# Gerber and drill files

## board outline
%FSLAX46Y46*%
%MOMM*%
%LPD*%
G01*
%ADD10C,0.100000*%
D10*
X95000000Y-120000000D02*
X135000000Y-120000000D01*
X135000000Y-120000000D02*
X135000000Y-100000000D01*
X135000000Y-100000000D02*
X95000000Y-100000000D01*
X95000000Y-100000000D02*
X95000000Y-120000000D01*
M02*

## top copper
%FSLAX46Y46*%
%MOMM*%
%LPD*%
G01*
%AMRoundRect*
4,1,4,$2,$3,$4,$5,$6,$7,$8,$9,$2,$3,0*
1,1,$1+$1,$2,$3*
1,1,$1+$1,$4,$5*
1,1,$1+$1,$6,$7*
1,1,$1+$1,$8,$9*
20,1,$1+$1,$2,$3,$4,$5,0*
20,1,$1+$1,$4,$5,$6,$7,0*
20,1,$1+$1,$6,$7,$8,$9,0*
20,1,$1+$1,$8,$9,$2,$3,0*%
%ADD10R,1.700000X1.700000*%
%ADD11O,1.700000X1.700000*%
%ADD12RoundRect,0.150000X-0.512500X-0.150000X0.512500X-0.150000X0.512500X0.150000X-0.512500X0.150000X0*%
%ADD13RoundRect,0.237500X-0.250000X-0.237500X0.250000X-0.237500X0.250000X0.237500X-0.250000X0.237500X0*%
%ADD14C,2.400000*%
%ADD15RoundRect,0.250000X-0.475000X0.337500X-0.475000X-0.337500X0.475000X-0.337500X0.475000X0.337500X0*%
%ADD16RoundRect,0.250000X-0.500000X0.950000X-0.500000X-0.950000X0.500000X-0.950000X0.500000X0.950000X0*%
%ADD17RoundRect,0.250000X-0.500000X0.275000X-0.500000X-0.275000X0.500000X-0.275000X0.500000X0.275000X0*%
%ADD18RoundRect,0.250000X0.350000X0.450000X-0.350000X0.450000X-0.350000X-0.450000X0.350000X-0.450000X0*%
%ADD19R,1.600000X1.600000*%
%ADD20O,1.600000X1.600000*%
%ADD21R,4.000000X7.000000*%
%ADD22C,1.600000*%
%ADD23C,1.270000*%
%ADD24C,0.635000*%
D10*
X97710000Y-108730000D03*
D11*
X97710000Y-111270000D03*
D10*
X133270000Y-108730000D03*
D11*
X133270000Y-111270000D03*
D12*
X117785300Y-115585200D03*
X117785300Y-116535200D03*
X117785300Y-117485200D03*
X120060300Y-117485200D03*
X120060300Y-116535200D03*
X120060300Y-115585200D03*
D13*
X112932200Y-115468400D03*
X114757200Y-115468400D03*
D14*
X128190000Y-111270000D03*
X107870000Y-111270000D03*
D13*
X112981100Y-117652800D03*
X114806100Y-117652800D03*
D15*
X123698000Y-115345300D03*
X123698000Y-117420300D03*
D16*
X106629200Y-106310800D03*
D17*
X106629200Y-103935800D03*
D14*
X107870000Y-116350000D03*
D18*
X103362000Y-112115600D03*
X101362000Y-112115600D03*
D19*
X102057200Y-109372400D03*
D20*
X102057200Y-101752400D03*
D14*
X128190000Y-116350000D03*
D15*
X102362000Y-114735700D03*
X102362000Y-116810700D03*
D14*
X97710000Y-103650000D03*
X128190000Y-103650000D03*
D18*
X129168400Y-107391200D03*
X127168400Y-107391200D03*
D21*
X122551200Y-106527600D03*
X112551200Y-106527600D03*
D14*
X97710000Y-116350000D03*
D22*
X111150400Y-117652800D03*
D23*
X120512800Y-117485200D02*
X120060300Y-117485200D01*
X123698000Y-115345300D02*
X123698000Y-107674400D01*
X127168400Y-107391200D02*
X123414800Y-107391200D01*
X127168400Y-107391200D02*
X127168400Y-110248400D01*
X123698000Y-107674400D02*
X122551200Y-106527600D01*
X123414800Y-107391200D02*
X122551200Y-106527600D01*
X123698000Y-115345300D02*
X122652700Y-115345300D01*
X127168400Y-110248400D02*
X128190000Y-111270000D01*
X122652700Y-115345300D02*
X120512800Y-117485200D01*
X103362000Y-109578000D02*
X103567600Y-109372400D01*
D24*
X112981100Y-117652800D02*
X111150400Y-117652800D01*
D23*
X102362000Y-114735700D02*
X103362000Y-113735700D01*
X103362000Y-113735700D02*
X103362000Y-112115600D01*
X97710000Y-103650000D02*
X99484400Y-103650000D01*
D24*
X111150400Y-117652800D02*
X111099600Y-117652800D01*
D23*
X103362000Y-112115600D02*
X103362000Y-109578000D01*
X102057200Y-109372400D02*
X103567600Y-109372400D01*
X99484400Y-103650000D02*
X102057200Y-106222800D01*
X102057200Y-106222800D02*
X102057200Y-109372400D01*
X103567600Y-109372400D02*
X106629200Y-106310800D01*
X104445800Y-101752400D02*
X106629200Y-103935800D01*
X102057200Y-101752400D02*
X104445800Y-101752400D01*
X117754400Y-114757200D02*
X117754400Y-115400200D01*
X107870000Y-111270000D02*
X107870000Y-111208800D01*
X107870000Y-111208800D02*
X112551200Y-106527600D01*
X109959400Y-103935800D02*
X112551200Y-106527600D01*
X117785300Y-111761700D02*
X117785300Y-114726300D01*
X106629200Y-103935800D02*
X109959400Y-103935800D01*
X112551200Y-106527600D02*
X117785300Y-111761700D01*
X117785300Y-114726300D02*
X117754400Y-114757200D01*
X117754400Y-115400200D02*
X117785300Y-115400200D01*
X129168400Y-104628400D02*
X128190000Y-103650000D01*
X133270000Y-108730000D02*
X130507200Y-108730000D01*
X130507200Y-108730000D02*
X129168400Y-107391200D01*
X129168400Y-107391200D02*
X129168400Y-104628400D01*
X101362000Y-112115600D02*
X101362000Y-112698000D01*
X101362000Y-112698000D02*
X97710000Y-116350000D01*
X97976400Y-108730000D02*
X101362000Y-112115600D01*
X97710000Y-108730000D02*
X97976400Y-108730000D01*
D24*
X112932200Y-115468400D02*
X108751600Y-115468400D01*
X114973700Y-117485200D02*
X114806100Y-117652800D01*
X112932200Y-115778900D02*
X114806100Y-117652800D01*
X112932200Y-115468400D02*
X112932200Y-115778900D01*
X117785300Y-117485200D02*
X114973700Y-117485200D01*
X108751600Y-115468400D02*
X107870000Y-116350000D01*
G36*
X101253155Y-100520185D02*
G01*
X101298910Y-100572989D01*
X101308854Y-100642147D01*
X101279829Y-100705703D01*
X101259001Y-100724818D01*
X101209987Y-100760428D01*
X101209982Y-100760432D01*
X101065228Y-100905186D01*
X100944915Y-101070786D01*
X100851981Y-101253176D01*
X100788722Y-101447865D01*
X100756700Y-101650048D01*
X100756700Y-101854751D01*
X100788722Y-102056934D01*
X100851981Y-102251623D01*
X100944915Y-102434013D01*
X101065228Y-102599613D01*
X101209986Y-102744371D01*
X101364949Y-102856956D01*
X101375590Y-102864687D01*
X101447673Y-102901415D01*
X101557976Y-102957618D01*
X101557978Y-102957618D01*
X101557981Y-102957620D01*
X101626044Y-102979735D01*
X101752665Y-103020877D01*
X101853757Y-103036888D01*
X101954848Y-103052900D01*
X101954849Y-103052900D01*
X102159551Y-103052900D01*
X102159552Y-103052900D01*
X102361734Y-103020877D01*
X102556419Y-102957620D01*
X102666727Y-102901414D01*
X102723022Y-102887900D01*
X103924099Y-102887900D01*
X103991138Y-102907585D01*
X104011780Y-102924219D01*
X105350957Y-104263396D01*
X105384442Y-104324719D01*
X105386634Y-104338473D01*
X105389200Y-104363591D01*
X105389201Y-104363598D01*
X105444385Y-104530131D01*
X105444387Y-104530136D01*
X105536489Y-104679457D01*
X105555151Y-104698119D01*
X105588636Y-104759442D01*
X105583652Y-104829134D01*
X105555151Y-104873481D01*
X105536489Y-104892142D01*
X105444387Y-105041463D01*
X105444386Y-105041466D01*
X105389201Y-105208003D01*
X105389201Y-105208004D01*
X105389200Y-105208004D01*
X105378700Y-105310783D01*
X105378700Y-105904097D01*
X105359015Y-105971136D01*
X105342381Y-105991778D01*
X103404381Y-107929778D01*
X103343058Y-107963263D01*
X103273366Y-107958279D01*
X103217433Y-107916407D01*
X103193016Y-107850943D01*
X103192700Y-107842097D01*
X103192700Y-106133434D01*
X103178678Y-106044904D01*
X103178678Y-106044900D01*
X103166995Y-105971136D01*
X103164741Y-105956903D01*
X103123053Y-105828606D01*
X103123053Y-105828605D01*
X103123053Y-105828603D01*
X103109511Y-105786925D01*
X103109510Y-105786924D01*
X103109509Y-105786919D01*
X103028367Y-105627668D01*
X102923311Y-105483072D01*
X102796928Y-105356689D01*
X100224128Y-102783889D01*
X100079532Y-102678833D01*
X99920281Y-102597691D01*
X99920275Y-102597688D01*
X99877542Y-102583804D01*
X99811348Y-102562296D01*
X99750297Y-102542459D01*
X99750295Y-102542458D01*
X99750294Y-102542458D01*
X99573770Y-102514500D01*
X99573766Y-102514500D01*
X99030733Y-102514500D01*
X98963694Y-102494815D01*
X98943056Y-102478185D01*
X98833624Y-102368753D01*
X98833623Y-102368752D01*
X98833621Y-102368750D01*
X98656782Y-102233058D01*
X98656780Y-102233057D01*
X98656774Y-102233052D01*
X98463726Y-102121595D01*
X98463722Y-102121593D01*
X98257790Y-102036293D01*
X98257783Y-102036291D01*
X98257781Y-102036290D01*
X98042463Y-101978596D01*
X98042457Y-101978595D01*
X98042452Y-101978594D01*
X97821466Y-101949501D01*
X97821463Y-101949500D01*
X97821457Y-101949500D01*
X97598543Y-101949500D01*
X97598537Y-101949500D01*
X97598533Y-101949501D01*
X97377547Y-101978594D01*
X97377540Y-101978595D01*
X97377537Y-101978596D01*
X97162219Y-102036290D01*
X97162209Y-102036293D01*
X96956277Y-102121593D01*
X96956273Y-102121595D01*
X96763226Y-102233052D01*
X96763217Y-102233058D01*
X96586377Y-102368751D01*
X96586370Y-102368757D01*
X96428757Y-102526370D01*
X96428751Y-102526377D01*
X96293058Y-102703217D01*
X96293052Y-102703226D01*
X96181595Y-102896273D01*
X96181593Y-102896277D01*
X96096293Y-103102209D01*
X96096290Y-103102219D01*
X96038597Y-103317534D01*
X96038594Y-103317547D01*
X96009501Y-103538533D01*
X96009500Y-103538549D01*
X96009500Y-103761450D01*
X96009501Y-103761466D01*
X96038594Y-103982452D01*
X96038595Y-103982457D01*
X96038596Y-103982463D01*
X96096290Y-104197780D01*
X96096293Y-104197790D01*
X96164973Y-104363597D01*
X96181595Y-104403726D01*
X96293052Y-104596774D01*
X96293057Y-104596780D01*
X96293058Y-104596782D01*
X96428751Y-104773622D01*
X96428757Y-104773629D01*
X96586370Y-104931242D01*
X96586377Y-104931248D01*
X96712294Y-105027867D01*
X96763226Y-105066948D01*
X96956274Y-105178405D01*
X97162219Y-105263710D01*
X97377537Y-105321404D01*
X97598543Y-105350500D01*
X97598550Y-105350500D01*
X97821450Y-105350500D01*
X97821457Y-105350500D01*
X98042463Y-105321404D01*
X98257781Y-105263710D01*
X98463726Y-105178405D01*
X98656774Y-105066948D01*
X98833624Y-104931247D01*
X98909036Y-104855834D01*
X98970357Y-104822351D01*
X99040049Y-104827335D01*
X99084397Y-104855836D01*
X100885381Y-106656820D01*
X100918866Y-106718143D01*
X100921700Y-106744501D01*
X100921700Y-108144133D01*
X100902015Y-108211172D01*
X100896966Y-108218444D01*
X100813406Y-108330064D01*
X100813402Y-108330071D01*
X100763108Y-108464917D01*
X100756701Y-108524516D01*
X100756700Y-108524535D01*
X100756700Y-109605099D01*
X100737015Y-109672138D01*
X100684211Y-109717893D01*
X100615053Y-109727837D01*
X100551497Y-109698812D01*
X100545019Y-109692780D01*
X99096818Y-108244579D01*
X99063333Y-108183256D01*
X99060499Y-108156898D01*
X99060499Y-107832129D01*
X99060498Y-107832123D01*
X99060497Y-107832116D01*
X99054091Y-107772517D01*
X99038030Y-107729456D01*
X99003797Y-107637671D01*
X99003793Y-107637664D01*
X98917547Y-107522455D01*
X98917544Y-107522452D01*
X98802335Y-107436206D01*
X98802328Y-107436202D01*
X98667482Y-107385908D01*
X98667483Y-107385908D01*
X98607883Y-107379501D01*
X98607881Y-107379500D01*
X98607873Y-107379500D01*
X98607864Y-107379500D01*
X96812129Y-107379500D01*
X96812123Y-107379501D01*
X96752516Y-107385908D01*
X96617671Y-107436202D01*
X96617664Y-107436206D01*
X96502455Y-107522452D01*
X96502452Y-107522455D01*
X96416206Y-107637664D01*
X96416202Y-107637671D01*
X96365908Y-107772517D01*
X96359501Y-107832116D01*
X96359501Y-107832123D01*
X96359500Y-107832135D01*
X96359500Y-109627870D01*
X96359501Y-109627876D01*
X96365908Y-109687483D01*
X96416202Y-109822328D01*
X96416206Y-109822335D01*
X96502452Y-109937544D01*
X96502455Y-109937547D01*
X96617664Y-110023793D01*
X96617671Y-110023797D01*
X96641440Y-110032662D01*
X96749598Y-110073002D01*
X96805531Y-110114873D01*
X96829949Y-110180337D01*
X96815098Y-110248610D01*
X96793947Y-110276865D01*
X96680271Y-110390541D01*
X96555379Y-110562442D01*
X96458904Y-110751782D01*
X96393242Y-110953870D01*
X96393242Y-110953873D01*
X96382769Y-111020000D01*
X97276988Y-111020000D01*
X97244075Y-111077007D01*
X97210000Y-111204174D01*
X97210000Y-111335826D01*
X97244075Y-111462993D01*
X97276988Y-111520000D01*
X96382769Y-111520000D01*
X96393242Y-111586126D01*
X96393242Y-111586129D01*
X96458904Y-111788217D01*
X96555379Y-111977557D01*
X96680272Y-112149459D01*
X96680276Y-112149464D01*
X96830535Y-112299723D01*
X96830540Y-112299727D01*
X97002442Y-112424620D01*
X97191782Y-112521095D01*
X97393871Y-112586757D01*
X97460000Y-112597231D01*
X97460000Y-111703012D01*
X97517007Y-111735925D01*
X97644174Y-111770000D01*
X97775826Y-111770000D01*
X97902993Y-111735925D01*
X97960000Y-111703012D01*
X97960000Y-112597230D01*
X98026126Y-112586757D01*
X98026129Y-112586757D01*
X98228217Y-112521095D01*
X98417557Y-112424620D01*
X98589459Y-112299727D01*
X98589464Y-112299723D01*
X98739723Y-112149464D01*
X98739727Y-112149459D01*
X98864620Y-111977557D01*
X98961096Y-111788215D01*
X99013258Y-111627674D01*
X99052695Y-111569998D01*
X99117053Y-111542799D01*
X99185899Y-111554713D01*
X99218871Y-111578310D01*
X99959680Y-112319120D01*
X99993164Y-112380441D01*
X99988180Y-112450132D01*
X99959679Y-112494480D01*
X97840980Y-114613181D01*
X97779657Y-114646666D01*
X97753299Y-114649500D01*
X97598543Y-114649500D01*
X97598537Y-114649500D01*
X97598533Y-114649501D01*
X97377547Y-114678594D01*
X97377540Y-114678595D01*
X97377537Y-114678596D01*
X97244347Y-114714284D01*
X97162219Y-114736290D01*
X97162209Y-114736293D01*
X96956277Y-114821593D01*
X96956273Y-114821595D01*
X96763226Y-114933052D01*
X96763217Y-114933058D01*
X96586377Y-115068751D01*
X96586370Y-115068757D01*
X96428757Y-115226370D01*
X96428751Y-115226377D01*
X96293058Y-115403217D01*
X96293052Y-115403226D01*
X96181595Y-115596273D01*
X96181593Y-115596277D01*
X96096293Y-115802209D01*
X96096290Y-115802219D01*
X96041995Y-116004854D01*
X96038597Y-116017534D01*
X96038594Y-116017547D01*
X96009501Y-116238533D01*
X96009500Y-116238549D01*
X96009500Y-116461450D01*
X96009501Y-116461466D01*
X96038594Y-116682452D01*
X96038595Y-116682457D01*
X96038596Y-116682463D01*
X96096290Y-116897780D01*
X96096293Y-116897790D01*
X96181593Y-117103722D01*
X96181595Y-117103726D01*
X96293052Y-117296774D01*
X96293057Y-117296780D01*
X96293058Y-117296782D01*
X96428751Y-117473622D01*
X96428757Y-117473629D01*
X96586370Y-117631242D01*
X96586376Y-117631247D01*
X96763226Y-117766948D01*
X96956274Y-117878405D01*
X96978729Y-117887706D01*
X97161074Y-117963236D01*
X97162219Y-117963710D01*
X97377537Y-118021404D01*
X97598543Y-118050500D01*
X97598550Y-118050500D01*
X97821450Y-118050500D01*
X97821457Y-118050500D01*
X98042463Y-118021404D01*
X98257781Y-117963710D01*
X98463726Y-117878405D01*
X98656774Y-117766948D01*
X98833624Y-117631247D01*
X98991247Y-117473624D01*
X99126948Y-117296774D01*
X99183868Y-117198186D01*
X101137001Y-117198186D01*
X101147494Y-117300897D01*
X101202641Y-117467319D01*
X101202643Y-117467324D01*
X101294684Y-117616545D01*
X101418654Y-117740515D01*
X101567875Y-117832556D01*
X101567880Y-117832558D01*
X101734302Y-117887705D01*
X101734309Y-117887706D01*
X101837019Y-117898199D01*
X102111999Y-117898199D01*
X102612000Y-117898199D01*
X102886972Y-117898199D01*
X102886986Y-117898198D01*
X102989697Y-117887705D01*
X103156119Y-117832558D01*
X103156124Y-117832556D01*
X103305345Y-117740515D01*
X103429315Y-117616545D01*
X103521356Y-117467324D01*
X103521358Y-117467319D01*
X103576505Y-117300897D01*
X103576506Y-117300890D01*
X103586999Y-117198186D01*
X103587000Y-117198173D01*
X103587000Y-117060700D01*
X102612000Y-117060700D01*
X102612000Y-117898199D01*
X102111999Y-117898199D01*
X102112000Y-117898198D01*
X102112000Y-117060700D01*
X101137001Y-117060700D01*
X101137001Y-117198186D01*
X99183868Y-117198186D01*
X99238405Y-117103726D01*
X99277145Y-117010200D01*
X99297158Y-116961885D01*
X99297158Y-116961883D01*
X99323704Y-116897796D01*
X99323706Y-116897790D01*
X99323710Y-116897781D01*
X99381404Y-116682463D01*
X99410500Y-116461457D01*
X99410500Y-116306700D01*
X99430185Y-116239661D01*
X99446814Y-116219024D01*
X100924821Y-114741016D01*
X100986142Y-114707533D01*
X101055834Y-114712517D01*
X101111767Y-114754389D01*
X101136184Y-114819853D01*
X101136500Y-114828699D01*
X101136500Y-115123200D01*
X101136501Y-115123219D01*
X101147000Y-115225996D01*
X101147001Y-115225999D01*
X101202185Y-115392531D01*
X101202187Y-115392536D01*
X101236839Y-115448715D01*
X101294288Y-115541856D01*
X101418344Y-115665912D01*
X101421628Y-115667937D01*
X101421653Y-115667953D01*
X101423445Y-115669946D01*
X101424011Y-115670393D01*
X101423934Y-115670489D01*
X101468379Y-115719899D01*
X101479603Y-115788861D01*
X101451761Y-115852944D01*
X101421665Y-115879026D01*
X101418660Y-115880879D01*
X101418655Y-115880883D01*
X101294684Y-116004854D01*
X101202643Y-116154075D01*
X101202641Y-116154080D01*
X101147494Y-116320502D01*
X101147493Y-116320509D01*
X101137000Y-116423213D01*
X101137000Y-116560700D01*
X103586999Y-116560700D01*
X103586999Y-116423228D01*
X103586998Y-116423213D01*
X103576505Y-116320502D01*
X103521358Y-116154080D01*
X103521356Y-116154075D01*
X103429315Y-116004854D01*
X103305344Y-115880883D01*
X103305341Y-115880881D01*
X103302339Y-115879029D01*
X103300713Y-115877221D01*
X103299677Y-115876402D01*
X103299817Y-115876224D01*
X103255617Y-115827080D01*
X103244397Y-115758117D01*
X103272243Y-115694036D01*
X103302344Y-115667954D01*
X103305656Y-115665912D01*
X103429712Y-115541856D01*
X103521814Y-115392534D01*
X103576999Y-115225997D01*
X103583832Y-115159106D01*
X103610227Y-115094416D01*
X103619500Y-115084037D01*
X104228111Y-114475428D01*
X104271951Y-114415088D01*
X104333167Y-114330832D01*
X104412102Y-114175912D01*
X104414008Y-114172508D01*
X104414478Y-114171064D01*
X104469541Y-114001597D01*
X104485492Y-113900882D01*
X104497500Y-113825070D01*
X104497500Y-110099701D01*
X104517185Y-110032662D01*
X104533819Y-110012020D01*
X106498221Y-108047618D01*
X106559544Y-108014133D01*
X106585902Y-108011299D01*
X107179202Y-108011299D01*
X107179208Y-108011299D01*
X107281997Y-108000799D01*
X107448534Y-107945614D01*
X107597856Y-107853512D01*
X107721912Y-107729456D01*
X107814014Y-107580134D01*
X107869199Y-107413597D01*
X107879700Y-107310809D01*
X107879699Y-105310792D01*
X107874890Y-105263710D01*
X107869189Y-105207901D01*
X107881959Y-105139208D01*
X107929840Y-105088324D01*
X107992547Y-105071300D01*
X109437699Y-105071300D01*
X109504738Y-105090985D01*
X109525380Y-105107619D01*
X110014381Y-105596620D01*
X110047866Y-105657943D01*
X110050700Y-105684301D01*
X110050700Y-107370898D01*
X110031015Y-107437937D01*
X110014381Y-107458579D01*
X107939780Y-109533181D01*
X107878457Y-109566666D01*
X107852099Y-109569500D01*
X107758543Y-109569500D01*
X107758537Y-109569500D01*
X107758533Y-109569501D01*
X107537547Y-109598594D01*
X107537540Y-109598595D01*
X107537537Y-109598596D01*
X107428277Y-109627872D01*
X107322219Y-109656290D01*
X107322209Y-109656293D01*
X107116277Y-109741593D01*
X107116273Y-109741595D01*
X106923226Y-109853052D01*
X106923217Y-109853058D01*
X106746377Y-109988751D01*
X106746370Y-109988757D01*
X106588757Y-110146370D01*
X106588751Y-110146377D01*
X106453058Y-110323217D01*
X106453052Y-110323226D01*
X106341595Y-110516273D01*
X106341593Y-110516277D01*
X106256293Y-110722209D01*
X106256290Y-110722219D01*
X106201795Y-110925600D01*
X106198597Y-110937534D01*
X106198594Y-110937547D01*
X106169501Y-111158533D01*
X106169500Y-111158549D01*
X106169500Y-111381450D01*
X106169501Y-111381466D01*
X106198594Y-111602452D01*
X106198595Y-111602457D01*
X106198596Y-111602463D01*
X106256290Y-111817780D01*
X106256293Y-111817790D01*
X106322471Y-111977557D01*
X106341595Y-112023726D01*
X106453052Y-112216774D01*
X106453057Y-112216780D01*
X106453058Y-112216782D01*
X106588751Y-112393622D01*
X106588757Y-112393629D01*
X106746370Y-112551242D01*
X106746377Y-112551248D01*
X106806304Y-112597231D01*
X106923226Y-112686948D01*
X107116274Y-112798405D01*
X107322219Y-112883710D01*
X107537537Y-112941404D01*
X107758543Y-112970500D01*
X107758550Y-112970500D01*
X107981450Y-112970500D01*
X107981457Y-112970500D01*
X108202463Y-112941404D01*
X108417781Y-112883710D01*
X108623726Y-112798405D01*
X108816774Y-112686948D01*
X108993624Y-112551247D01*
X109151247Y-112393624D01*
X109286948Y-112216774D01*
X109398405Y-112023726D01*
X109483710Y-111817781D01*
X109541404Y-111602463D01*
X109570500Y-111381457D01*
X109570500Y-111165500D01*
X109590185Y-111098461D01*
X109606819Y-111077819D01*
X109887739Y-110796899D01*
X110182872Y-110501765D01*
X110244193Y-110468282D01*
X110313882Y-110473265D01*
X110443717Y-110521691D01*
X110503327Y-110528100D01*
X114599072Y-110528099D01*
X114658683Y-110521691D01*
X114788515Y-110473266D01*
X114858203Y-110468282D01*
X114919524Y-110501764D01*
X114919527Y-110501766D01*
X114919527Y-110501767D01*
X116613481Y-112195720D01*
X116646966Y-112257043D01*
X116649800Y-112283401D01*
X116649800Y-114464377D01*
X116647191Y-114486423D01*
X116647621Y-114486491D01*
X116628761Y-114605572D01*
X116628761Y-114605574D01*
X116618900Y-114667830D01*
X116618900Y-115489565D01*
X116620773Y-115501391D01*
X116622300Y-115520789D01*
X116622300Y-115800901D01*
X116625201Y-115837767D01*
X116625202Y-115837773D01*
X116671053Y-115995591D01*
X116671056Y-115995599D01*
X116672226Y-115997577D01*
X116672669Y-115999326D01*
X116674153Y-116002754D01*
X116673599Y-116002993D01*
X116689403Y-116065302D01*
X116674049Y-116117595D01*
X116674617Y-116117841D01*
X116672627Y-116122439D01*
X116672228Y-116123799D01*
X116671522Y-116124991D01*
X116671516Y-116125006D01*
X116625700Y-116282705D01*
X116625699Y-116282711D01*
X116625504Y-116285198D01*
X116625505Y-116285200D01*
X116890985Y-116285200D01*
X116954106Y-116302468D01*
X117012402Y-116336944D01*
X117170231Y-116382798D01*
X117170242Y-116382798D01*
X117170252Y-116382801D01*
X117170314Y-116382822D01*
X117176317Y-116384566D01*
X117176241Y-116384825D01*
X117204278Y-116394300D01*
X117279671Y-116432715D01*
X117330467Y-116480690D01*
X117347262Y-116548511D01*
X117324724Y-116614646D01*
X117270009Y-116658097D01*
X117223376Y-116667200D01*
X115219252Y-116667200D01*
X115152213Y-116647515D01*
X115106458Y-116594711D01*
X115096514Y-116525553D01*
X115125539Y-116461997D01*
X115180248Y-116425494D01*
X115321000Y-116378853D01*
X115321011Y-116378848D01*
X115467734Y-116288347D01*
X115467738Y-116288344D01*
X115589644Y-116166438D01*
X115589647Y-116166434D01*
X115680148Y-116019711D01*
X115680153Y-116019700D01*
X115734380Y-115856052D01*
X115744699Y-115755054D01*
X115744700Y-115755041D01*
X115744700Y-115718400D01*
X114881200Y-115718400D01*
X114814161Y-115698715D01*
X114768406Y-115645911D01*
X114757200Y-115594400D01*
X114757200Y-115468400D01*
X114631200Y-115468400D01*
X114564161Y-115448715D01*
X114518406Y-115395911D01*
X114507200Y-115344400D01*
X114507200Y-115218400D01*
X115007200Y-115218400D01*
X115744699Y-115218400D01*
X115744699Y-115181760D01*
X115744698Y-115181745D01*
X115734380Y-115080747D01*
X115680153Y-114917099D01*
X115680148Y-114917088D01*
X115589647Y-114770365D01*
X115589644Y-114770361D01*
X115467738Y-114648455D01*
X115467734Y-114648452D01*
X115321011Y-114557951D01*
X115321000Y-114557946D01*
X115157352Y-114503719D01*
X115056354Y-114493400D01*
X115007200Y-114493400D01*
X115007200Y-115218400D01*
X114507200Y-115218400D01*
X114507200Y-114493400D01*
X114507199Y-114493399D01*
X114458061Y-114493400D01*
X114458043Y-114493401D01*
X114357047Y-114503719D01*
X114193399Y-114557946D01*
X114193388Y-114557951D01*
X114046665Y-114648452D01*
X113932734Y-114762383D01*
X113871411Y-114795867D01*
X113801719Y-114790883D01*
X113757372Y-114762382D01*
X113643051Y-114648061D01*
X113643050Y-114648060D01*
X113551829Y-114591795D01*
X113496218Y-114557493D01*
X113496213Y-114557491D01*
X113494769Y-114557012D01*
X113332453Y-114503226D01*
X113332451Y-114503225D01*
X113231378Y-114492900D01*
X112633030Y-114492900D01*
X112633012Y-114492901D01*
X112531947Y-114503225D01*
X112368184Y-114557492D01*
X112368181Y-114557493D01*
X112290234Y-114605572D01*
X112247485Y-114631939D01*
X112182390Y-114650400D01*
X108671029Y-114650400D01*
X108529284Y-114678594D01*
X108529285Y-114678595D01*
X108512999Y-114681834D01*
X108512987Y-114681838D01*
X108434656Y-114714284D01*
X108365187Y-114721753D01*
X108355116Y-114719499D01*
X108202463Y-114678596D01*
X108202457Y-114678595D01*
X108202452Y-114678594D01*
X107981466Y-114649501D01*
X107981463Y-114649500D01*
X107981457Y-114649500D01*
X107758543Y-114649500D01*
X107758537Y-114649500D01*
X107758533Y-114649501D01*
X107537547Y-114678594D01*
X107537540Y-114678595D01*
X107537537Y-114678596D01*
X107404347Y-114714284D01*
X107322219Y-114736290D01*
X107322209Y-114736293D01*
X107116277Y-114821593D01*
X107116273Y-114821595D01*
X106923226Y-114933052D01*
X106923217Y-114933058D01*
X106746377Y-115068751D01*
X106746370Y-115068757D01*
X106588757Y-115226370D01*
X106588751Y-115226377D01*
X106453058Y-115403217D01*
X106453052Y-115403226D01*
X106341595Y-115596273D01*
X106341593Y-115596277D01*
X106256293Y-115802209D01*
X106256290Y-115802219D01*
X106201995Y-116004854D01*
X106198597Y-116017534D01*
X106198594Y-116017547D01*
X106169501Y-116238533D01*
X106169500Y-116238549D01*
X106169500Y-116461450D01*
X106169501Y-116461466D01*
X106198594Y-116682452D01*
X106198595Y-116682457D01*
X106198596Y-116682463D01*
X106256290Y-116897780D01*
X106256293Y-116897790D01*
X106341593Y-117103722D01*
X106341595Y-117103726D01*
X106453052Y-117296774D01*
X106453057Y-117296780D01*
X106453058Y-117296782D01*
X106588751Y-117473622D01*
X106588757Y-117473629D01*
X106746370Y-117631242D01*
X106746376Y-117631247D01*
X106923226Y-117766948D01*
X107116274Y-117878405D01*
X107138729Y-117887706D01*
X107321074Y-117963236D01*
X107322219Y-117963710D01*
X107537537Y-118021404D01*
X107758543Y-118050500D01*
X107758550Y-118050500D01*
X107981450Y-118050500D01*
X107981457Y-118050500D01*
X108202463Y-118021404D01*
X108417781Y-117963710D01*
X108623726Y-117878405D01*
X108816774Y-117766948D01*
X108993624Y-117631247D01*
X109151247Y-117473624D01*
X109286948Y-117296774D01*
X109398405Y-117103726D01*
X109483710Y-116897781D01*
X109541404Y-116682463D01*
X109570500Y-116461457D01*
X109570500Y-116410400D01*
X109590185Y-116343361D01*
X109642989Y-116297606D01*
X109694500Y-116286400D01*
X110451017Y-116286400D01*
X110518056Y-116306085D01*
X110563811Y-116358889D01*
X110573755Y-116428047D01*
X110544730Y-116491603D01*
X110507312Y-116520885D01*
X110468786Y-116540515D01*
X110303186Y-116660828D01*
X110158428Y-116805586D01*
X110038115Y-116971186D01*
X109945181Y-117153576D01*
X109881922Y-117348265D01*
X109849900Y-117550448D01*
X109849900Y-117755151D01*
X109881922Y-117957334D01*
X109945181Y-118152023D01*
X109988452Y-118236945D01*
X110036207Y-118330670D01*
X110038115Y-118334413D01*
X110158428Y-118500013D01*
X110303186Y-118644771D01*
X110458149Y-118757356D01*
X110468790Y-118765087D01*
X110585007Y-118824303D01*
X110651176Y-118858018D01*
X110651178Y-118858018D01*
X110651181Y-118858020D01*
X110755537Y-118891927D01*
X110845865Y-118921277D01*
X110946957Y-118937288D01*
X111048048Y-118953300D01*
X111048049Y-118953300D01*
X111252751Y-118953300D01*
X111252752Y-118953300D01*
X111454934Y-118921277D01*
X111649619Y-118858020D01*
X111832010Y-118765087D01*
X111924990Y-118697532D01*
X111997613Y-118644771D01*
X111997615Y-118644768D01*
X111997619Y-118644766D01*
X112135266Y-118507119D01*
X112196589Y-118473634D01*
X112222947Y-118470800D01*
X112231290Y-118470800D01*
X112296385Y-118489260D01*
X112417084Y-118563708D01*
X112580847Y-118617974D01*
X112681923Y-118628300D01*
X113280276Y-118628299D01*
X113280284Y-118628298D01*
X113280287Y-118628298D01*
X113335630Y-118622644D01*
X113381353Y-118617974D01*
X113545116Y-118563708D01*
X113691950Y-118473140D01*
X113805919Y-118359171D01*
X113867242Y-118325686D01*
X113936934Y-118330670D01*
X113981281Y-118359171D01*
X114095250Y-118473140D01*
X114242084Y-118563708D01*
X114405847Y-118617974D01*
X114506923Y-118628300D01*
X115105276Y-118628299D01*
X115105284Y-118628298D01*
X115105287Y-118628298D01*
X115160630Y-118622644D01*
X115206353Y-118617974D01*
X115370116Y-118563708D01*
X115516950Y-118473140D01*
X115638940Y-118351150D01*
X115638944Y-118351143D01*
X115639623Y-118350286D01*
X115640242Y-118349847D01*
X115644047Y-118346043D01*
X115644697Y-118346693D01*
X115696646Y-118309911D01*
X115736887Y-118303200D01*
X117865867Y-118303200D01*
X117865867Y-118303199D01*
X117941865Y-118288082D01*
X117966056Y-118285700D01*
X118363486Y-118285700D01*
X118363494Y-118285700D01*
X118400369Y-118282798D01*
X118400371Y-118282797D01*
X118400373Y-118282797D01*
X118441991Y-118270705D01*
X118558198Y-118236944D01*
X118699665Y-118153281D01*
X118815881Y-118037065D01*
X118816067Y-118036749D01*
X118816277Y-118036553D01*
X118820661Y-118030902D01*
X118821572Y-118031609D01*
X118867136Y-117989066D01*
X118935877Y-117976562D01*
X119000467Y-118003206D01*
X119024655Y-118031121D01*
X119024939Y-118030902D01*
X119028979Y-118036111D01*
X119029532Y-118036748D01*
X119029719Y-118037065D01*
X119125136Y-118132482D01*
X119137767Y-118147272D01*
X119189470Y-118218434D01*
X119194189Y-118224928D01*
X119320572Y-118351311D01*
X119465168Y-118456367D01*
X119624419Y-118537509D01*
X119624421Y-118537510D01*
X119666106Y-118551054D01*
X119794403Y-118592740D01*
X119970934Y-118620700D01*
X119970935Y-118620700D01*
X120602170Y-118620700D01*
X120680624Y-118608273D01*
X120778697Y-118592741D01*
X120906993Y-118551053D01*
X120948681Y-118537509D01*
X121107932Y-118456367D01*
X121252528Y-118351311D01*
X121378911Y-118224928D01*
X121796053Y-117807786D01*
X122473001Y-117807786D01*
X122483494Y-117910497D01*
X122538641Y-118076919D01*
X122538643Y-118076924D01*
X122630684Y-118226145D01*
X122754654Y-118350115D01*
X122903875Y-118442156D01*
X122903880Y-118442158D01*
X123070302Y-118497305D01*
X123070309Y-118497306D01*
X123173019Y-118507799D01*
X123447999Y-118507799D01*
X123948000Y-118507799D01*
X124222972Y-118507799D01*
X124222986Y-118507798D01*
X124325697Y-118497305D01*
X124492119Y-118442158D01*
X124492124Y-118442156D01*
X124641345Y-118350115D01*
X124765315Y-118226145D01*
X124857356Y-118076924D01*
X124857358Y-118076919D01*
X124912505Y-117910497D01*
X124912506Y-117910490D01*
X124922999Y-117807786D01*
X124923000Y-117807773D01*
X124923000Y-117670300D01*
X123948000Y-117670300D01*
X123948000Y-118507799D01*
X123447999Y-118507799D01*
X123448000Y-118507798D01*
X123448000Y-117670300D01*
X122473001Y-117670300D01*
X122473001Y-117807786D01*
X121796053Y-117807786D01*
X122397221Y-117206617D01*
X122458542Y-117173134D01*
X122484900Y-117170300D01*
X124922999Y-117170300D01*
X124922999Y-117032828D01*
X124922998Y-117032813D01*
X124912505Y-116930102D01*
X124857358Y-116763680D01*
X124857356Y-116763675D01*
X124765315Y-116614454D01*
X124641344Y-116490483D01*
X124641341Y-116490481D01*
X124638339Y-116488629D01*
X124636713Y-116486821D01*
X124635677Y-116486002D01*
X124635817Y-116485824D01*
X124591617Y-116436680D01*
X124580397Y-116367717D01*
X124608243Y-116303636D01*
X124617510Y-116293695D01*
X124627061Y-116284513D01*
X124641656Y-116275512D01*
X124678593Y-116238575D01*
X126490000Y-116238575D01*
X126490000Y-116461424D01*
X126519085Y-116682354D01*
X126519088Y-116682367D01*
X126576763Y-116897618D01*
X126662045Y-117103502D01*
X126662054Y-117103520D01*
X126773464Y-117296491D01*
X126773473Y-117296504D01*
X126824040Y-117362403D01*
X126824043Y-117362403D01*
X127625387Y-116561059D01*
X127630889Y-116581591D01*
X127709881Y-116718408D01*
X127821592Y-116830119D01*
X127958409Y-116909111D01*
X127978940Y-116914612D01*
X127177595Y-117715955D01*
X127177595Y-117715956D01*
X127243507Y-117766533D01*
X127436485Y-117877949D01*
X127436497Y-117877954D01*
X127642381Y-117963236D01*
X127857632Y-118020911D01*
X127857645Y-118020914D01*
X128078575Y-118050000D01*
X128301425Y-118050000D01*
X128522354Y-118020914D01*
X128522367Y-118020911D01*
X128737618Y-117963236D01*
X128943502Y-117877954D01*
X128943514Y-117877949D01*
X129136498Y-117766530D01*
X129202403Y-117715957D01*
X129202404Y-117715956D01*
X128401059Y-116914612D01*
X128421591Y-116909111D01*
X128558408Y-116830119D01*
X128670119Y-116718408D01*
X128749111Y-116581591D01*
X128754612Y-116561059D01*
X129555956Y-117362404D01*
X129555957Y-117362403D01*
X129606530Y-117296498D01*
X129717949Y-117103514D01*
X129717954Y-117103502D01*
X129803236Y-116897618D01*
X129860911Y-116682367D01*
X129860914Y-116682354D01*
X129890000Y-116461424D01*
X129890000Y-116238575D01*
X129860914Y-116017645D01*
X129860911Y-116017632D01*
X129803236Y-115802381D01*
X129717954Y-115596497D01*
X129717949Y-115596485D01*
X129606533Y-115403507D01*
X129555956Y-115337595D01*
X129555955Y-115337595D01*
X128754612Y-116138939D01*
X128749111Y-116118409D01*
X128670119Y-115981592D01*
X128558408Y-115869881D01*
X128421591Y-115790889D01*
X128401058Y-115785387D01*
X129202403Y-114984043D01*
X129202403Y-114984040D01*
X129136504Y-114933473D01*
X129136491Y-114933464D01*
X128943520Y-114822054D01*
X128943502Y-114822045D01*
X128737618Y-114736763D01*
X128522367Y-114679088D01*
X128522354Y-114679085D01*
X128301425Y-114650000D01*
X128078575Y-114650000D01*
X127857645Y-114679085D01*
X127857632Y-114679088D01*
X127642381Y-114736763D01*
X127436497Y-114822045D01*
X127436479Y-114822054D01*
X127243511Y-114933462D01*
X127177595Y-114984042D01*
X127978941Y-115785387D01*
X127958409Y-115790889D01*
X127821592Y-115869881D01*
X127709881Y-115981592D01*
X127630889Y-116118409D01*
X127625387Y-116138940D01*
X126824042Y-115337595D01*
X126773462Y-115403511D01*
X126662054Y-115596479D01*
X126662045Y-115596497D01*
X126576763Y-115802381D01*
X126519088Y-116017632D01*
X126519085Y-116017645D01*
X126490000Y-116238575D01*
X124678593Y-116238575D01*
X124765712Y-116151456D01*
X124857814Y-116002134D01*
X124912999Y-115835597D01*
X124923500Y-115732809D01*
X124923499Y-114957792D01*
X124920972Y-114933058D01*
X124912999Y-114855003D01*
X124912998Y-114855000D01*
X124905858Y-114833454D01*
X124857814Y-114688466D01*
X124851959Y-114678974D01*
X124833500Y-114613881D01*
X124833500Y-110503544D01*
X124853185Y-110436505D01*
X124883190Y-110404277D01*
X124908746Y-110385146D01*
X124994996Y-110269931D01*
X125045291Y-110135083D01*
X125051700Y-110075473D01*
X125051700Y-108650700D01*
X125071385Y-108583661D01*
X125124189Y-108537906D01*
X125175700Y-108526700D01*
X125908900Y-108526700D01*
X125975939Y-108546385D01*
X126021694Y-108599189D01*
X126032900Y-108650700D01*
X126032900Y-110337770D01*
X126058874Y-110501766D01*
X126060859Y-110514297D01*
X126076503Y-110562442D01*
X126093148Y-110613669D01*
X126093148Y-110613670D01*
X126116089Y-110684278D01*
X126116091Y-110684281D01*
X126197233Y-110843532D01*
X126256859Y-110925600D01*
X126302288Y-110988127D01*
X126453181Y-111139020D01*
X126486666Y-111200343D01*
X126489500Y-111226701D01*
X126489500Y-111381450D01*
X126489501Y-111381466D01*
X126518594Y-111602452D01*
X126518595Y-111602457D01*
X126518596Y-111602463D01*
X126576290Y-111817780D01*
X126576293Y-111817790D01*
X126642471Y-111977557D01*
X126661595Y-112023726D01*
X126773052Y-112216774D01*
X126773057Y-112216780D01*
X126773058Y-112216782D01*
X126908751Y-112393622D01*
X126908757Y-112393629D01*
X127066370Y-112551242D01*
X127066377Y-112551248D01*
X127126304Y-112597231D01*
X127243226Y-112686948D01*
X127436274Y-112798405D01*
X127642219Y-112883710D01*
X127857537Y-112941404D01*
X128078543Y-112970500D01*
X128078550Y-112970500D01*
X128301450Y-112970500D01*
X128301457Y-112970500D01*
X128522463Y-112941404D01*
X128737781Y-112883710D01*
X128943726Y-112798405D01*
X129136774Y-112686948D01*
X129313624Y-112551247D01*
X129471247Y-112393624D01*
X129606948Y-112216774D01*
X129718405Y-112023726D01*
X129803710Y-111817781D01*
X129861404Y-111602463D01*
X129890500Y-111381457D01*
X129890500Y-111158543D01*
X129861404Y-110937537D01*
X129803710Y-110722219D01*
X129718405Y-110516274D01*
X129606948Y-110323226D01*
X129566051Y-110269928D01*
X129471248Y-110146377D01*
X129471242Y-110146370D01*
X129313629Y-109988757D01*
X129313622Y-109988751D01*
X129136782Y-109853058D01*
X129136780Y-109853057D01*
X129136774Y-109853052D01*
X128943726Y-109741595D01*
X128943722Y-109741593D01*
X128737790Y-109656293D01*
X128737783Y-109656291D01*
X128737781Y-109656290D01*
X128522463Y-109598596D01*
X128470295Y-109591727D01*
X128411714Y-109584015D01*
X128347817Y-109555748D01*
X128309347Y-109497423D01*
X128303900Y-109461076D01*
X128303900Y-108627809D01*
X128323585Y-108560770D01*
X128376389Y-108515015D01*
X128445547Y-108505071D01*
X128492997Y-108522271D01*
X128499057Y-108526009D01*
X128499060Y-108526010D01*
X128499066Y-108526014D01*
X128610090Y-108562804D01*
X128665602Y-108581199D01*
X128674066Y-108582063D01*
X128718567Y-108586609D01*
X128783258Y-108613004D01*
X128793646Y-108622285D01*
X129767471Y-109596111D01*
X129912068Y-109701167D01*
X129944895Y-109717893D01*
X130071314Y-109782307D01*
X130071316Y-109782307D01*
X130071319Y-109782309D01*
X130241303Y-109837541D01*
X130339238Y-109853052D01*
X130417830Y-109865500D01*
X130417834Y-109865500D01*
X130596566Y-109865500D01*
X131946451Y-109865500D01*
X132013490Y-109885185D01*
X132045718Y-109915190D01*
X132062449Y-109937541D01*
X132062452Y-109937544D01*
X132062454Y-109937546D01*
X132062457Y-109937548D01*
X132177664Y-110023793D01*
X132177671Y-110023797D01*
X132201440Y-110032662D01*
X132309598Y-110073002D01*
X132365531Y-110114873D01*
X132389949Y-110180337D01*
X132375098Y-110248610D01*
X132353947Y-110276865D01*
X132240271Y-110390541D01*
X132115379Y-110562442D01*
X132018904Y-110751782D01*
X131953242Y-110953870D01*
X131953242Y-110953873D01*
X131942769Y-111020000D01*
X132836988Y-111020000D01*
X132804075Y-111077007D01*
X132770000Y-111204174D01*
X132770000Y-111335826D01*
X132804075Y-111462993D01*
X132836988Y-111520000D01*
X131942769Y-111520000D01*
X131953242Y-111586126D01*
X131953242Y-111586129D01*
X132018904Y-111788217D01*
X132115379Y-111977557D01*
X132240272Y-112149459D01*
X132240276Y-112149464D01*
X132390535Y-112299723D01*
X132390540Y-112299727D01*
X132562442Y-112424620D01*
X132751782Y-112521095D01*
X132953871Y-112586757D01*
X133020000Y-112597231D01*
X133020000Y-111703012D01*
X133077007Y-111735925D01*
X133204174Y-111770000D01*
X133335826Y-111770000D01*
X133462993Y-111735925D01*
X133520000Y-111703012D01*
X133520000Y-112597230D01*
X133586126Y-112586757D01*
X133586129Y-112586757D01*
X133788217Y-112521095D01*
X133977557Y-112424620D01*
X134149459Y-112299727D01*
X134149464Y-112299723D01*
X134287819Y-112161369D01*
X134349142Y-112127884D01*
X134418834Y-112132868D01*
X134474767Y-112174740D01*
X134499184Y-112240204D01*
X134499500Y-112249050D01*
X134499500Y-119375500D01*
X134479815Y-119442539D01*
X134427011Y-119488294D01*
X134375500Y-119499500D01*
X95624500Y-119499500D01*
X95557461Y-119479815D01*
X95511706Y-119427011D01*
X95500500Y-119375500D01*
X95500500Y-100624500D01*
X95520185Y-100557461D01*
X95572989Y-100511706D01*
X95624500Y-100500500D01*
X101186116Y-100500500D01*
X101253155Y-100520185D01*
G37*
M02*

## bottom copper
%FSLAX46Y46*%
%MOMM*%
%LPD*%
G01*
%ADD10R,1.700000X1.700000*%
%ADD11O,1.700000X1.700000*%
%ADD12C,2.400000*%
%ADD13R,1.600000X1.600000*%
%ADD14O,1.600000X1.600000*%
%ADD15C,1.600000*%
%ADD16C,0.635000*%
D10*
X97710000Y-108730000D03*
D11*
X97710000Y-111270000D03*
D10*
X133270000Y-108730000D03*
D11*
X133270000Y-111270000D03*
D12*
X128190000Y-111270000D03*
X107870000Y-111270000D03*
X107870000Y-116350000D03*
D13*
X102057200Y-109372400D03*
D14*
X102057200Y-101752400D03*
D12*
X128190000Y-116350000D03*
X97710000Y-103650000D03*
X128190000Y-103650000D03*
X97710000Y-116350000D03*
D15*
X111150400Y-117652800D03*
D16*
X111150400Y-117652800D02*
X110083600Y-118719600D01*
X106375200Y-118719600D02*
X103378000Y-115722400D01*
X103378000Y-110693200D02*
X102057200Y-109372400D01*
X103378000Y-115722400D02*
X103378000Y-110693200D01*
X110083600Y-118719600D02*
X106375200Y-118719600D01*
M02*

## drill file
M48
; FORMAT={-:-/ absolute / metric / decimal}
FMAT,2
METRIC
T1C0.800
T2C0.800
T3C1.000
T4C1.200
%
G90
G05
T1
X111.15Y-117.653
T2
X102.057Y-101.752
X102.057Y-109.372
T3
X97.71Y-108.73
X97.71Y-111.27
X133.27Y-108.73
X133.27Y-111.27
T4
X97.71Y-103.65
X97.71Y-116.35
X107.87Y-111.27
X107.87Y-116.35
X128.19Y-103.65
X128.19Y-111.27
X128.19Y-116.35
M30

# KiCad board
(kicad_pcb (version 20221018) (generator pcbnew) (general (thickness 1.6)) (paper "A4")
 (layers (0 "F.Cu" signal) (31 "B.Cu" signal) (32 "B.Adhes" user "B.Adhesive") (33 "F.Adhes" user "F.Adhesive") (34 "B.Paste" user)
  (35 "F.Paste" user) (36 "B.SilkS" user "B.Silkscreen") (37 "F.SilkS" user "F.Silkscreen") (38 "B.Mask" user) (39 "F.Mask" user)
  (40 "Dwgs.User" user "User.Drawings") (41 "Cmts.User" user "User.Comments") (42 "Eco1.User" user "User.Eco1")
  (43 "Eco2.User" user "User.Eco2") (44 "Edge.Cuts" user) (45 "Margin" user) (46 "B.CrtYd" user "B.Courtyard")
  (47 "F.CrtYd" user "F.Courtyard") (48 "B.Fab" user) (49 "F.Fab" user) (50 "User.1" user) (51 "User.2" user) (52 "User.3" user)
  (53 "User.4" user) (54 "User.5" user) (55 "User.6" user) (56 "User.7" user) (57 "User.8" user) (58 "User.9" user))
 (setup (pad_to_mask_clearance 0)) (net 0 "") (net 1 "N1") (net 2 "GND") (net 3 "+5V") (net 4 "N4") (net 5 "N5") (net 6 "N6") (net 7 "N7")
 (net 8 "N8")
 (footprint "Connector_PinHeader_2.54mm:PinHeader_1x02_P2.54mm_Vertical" (layer "F.Cu") (at 97.71 108.73)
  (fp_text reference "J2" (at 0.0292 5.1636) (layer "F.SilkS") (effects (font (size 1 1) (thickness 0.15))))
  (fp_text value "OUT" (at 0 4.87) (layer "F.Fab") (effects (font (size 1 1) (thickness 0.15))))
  (pad "1" thru_hole rect (at 0 0) (size 1.7 1.7) (drill 1) (layers "*.Cu" "*.Mask") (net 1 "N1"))
  (pad "2" thru_hole oval (at 0 2.54) (size 1.7 1.7) (drill 1) (layers "*.Cu" "*.Mask") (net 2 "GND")))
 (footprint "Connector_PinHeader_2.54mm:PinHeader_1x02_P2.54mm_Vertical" (layer "F.Cu") (at 133.27 108.73)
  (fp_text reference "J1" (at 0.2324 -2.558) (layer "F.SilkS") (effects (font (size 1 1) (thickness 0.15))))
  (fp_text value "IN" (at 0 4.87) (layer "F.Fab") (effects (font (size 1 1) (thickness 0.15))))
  (pad "1" thru_hole rect (at 0 0) (size 1.7 1.7) (drill 1) (layers "*.Cu" "*.Mask") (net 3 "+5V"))
  (pad "2" thru_hole oval (at 0 2.54) (size 1.7 1.7) (drill 1) (layers "*.Cu" "*.Mask") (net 2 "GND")))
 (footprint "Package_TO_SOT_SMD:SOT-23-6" (layer "F.Cu") (at 118.9228 116.5352)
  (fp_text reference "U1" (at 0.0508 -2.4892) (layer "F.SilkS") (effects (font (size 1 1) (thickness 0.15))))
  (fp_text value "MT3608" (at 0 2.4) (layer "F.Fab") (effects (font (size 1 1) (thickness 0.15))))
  (pad "1" smd roundrect (at -1.1375 -0.95) (size 1.325 0.6) (layers "F.Cu" "F.Paste" "F.Mask") (roundrect_rratio 0.25) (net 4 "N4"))
  (pad "2" smd roundrect (at -1.1375 0) (size 1.325 0.6) (layers "F.Cu" "F.Paste" "F.Mask") (roundrect_rratio 0.25) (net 2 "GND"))
  (pad "3" smd roundrect (at -1.1375 0.95) (size 1.325 0.6) (layers "F.Cu" "F.Paste" "F.Mask") (roundrect_rratio 0.25) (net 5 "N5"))
  (pad "4" smd roundrect (at 1.1375 0.95) (size 1.325 0.6) (layers "F.Cu" "F.Paste" "F.Mask") (roundrect_rratio 0.25) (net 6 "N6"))
  (pad "5" smd roundrect (at 1.1375 0) (size 1.325 0.6) (layers "F.Cu" "F.Paste" "F.Mask") (roundrect_rratio 0.25) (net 6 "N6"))
  (pad "6" smd roundrect (at 1.1375 -0.95) (size 1.325 0.6) (layers "F.Cu" "F.Paste" "F.Mask") (roundrect_rratio 0.25) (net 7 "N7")))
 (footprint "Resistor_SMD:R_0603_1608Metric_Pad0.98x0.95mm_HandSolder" (layer "F.Cu") (at 113.8447 115.4684)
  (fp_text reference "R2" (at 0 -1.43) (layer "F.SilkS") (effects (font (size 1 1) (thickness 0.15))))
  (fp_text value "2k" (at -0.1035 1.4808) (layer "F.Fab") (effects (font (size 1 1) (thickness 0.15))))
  (pad "1" smd roundrect (at -0.9125 0) (size 0.975 0.95) (layers "F.Cu" "F.Paste" "F.Mask") (roundrect_rratio 0.25) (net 5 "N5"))
  (pad "2" smd roundrect (at 0.9125 0) (size 0.975 0.95) (layers "F.Cu" "F.Paste" "F.Mask") (roundrect_rratio 0.25) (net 2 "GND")))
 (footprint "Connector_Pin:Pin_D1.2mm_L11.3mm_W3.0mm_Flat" (layer "F.Cu") (at 128.19 111.27)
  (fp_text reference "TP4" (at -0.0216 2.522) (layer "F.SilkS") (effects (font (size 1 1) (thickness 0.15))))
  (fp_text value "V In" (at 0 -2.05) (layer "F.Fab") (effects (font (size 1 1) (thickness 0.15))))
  (pad "1" thru_hole circle (at 0 0) (size 2.4 2.4) (drill 1.2) (layers "*.Cu" "*.Mask") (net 6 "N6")))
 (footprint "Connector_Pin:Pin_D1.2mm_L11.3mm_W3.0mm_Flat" (layer "F.Cu") (at 107.87 111.27)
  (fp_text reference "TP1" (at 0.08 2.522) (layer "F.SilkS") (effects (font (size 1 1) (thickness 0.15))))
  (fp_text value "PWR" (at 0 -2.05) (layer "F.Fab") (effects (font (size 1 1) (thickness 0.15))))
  (pad "1" thru_hole circle (at 0 0) (size 2.4 2.4) (drill 1.2) (layers "*.Cu" "*.Mask") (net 4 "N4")))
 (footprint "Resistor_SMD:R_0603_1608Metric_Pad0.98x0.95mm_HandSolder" (layer "F.Cu") (at 113.8936 117.6528)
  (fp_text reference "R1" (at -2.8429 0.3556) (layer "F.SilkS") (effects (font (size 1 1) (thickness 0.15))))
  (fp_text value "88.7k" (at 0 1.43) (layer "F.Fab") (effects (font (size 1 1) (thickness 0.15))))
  (pad "1" smd roundrect (at -0.9125 0) (size 0.975 0.95) (layers "F.Cu" "F.Paste" "F.Mask") (roundrect_rratio 0.25) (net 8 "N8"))
  (pad "2" smd roundrect (at 0.9125 0) (size 0.975 0.95) (layers "F.Cu" "F.Paste" "F.Mask") (roundrect_rratio 0.25) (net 5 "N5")))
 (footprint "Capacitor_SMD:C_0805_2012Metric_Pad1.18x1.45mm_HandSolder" (layer "F.Cu") (at 123.698 116.3828 -90)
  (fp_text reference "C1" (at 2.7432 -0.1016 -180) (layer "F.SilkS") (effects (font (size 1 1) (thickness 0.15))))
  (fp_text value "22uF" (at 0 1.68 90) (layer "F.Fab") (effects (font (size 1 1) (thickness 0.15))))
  (pad "1" smd roundrect (at -1.0375 0 270) (size 1.175 1.45) (layers "F.Cu" "F.Paste" "F.Mask") (roundrect_rratio 0.212766) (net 6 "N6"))
  (pad "2" smd roundrect (at 1.0375 0 270) (size 1.175 1.45) (layers "F.Cu" "F.Paste" "F.Mask") (roundrect_rratio 0.212766) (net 2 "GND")))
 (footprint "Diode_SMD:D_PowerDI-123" (layer "F.Cu") (at 106.6292 105.4608 90)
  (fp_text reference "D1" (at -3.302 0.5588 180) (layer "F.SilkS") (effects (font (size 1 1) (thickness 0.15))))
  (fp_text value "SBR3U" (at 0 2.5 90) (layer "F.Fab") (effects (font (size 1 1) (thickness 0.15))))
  (pad "1" smd roundrect (at -0.85 0 270) (size 2.4 1.5) (layers "F.Cu" "F.Paste" "F.Mask") (roundrect_rratio 0.1666666667) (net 8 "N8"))
  (pad "2" smd roundrect (at 1.525 0 270) (size 1.05 1.5) (layers "F.Cu" "F.Paste" "F.Mask") (roundrect_rratio 0.2380952381) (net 4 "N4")))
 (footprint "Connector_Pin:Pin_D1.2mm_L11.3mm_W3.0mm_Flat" (layer "F.Cu") (at 107.87 116.35)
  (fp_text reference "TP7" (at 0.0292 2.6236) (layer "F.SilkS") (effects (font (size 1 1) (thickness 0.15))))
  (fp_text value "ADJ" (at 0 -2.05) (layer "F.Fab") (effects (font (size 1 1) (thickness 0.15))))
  (pad "1" thru_hole circle (at 0 0) (size 2.4 2.4) (drill 1.2) (layers "*.Cu" "*.Mask") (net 5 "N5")))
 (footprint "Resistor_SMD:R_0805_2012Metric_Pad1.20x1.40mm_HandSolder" (layer "F.Cu") (at 102.362 112.1156 180)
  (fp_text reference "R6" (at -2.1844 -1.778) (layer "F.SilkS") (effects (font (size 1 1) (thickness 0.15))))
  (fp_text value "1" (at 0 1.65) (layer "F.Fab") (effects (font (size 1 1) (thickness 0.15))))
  (pad "1" smd roundrect (at -1 0 180) (size 1.2 1.4) (layers "F.Cu" "F.Paste" "F.Mask") (roundrect_rratio 0.208333) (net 8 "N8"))
  (pad "2" smd roundrect (at 1 0 180) (size 1.2 1.4) (layers "F.Cu" "F.Paste" "F.Mask") (roundrect_rratio 0.208333) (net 1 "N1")))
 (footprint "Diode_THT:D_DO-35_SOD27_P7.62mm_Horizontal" (layer "F.Cu") (at 102.0572 109.3724 90)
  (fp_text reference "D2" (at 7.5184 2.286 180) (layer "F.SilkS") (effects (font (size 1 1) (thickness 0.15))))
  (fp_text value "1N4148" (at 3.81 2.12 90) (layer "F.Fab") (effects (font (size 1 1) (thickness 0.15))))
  (pad "1" thru_hole rect (at 0 0 90) (size 1.6 1.6) (drill 0.8) (layers "*.Cu" "*.Mask") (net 8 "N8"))
  (pad "2" thru_hole oval (at 7.62 0 90) (size 1.6 1.6) (drill 0.8) (layers "*.Cu" "*.Mask") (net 4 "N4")))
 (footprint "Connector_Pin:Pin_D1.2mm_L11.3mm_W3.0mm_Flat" (layer "F.Cu") (at 128.19 116.35)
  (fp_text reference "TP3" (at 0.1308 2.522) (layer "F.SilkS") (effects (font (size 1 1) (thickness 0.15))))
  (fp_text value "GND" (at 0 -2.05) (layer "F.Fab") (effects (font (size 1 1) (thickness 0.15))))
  (pad "1" thru_hole circle (at 0 0) (size 2.4 2.4) (drill 1.2) (layers "*.Cu" "*.Mask") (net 2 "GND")))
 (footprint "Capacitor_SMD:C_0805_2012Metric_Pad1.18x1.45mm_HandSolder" (layer "F.Cu") (at 102.362 115.7732 -90)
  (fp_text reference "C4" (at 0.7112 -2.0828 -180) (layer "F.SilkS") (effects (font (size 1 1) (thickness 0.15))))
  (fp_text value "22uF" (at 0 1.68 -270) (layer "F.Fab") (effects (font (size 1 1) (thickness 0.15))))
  (pad "1" smd roundrect (at -1.0375 0 270) (size 1.175 1.45) (layers "F.Cu" "F.Paste" "F.Mask") (roundrect_rratio 0.212766) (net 8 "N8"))
  (pad "2" smd roundrect (at 1.0375 0 270) (size 1.175 1.45) (layers "F.Cu" "F.Paste" "F.Mask") (roundrect_rratio 0.212766) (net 2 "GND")))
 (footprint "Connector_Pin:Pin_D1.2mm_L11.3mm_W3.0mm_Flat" (layer "F.Cu") (at 97.71 103.65)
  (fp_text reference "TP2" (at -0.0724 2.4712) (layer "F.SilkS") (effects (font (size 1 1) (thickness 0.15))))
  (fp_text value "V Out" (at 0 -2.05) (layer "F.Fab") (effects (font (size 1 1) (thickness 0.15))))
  (pad "1" thru_hole circle (at 0 0) (size 2.4 2.4) (drill 1.2) (layers "*.Cu" "*.Mask") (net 8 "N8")))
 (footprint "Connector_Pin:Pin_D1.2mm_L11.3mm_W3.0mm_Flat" (layer "F.Cu") (at 128.19 103.65)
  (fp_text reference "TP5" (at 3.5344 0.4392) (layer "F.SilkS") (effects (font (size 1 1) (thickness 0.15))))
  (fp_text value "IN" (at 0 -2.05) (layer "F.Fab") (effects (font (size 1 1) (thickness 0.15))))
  (pad "1" thru_hole circle (at 0 0) (size 2.4 2.4) (drill 1.2) (layers "*.Cu" "*.Mask") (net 3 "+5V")))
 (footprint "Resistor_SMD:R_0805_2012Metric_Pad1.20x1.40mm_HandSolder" (layer "F.Cu") (at 128.1684 107.3912 180)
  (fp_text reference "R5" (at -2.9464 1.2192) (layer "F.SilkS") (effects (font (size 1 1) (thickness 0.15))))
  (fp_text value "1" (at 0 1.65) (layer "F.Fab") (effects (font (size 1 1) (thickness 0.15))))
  (pad "1" smd roundrect (at -1 0 180) (size 1.2 1.4) (layers "F.Cu" "F.Paste" "F.Mask") (roundrect_rratio 0.208333) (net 3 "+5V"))
  (pad "2" smd roundrect (at 1 0 180) (size 1.2 1.4) (layers "F.Cu" "F.Paste" "F.Mask") (roundrect_rratio 0.208333) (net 6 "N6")))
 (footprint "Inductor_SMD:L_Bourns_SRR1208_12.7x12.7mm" (layer "F.Cu") (at 117.5512 106.5276 180)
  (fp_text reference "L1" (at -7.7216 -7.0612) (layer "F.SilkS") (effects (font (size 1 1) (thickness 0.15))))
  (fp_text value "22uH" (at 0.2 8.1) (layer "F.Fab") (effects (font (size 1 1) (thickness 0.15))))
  (pad "1" smd rect (at -5 0 180) (size 4 7) (layers "F.Cu" "F.Paste" "F.Mask") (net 6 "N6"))
  (pad "2" smd rect (at 5 0 180) (size 4 7) (layers "F.Cu" "F.Paste" "F.Mask") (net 4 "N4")))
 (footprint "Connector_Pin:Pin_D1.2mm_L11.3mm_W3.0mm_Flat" (layer "F.Cu") (at 97.71 116.35)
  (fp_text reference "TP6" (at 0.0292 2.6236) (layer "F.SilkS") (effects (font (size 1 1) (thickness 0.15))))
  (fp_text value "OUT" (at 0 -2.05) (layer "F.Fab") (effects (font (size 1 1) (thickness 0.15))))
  (pad "1" thru_hole circle (at 0 0) (size 2.4 2.4) (drill 1.2) (layers "*.Cu" "*.Mask") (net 1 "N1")))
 (gr_line (start 95 120) (end 135 120) (stroke (width 0.1) (type default)) (layer "Edge.Cuts"))
 (gr_line (start 135 120) (end 135 100) (stroke (width 0.1) (type default)) (layer "Edge.Cuts"))
 (gr_line (start 135 100) (end 95 100) (stroke (width 0.1) (type default)) (layer "Edge.Cuts"))
 (gr_line (start 95 100) (end 95 120) (stroke (width 0.1) (type default)) (layer "Edge.Cuts"))
 (segment (start 120.5128 117.4852) (end 120.0603 117.4852) (width 1.27) (layer "F.Cu") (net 6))
 (segment (start 123.698 115.3453) (end 123.698 107.6744) (width 1.27) (layer "F.Cu") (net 6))
 (segment (start 127.1684 107.3912) (end 123.4148 107.3912) (width 1.27) (layer "F.Cu") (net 6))
 (segment (start 127.1684 107.3912) (end 127.1684 110.2484) (width 1.27) (layer "F.Cu") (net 6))
 (segment (start 123.698 107.6744) (end 122.5512 106.5276) (width 1.27) (layer "F.Cu") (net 6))
 (segment (start 123.4148 107.3912) (end 122.5512 106.5276) (width 1.27) (layer "F.Cu") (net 6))
 (segment (start 123.698 115.3453) (end 122.6527 115.3453) (width 1.27) (layer "F.Cu") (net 6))
 (segment (start 127.1684 110.2484) (end 128.19 111.27) (width 1.27) (layer "F.Cu") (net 6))
 (segment (start 122.6527 115.3453) (end 120.5128 117.4852) (width 1.27) (layer "F.Cu") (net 6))
 (segment (start 103.362 109.578) (end 103.5676 109.3724) (width 1.27) (layer "F.Cu") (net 8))
 (segment (start 112.9811 117.6528) (end 111.1504 117.6528) (width 0.635) (layer "F.Cu") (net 8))
 (segment (start 102.362 114.7357) (end 103.362 113.7357) (width 1.27) (layer "F.Cu") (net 8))
 (segment (start 103.362 113.7357) (end 103.362 112.1156) (width 1.27) (layer "F.Cu") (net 8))
 (segment (start 97.71 103.65) (end 99.4844 103.65) (width 1.27) (layer "F.Cu") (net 8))
 (segment (start 111.1504 117.6528) (end 111.0996 117.6528) (width 0.635) (layer "F.Cu") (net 8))
 (segment (start 103.362 112.1156) (end 103.362 109.578) (width 1.27) (layer "F.Cu") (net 8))
 (segment (start 102.0572 109.3724) (end 103.5676 109.3724) (width 1.27) (layer "F.Cu") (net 8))
 (segment (start 99.4844 103.65) (end 102.0572 106.2228) (width 1.27) (layer "F.Cu") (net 8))
 (segment (start 102.0572 106.2228) (end 102.0572 109.3724) (width 1.27) (layer "F.Cu") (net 8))
 (segment (start 103.5676 109.3724) (end 106.6292 106.3108) (width 1.27) (layer "F.Cu") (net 8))
 (via (at 111.1504 117.6528) (size 1.6) (drill 0.8) (layers "F.Cu" "B.Cu") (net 8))
 (segment (start 111.1504 117.6528) (end 110.0836 118.7196) (width 0.635) (layer "B.Cu") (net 8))
 (segment (start 106.3752 118.7196) (end 103.378 115.7224) (width 0.635) (layer "B.Cu") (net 8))
 (segment (start 103.378 110.6932) (end 102.0572 109.3724) (width 0.635) (layer "B.Cu") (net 8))
 (segment (start 103.378 115.7224) (end 103.378 110.6932) (width 0.635) (layer "B.Cu") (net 8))
 (segment (start 110.0836 118.7196) (end 106.3752 118.7196) (width 0.635) (layer "B.Cu") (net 8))
 (segment (start 104.4458 101.7524) (end 106.6292 103.9358) (width 1.27) (layer "F.Cu") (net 4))
 (segment (start 102.0572 101.7524) (end 104.4458 101.7524) (width 1.27) (layer "F.Cu") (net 4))
 (segment (start 117.7544 114.7572) (end 117.7544 115.4002) (width 1.27) (layer "F.Cu") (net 4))
 (segment (start 107.87 111.27) (end 107.87 111.2088) (width 1.27) (layer "F.Cu") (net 4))
 (segment (start 107.87 111.2088) (end 112.5512 106.5276) (width 1.27) (layer "F.Cu") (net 4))
 (segment (start 109.9594 103.9358) (end 112.5512 106.5276) (width 1.27) (layer "F.Cu") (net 4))
 (segment (start 117.7853 111.7617) (end 117.7853 114.7263) (width 1.27) (layer "F.Cu") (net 4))
 (segment (start 106.6292 103.9358) (end 109.9594 103.9358) (width 1.27) (layer "F.Cu") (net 4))
 (segment (start 112.5512 106.5276) (end 117.7853 111.7617) (width 1.27) (layer "F.Cu") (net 4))
 (segment (start 117.7853 114.7263) (end 117.7544 114.7572) (width 1.27) (layer "F.Cu") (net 4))
 (segment (start 117.7544 115.4002) (end 117.7853 115.4002) (width 1.27) (layer "F.Cu") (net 4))
 (segment (start 129.1684 104.6284) (end 128.19 103.65) (width 1.27) (layer "F.Cu") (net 3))
 (segment (start 133.27 108.73) (end 130.5072 108.73) (width 1.27) (layer "F.Cu") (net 3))
 (segment (start 130.5072 108.73) (end 129.1684 107.3912) (width 1.27) (layer "F.Cu") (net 3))
 (segment (start 129.1684 107.3912) (end 129.1684 104.6284) (width 1.27) (layer "F.Cu") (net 3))
 (segment (start 101.362 112.1156) (end 101.362 112.698) (width 1.27) (layer "F.Cu") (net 1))
 (segment (start 101.362 112.698) (end 97.71 116.35) (width 1.27) (layer "F.Cu") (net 1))
 (segment (start 97.9764 108.73) (end 101.362 112.1156) (width 1.27) (layer "F.Cu") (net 1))
 (segment (start 97.71 108.73) (end 97.9764 108.73) (width 1.27) (layer "F.Cu") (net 1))
 (segment (start 112.9322 115.4684) (end 108.7516 115.4684) (width 0.635) (layer "F.Cu") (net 5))
 (segment (start 114.9737 117.4852) (end 114.8061 117.6528) (width 0.635) (layer "F.Cu") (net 5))
 (segment (start 112.9322 115.7789) (end 114.8061 117.6528) (width 0.635) (layer "F.Cu") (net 5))
 (segment (start 112.9322 115.4684) (end 112.9322 115.7789) (width 0.635) (layer "F.Cu") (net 5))
 (segment (start 117.7853 117.4852) (end 114.9737 117.4852) (width 0.635) (layer "F.Cu") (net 5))
 (segment (start 108.7516 115.4684) (end 107.87 116.35) (width 0.635) (layer "F.Cu") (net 5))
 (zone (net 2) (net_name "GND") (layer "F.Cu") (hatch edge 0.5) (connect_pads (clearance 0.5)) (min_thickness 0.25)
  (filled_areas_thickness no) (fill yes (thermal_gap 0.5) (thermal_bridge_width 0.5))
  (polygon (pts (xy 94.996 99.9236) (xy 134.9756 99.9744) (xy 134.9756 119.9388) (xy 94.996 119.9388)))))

